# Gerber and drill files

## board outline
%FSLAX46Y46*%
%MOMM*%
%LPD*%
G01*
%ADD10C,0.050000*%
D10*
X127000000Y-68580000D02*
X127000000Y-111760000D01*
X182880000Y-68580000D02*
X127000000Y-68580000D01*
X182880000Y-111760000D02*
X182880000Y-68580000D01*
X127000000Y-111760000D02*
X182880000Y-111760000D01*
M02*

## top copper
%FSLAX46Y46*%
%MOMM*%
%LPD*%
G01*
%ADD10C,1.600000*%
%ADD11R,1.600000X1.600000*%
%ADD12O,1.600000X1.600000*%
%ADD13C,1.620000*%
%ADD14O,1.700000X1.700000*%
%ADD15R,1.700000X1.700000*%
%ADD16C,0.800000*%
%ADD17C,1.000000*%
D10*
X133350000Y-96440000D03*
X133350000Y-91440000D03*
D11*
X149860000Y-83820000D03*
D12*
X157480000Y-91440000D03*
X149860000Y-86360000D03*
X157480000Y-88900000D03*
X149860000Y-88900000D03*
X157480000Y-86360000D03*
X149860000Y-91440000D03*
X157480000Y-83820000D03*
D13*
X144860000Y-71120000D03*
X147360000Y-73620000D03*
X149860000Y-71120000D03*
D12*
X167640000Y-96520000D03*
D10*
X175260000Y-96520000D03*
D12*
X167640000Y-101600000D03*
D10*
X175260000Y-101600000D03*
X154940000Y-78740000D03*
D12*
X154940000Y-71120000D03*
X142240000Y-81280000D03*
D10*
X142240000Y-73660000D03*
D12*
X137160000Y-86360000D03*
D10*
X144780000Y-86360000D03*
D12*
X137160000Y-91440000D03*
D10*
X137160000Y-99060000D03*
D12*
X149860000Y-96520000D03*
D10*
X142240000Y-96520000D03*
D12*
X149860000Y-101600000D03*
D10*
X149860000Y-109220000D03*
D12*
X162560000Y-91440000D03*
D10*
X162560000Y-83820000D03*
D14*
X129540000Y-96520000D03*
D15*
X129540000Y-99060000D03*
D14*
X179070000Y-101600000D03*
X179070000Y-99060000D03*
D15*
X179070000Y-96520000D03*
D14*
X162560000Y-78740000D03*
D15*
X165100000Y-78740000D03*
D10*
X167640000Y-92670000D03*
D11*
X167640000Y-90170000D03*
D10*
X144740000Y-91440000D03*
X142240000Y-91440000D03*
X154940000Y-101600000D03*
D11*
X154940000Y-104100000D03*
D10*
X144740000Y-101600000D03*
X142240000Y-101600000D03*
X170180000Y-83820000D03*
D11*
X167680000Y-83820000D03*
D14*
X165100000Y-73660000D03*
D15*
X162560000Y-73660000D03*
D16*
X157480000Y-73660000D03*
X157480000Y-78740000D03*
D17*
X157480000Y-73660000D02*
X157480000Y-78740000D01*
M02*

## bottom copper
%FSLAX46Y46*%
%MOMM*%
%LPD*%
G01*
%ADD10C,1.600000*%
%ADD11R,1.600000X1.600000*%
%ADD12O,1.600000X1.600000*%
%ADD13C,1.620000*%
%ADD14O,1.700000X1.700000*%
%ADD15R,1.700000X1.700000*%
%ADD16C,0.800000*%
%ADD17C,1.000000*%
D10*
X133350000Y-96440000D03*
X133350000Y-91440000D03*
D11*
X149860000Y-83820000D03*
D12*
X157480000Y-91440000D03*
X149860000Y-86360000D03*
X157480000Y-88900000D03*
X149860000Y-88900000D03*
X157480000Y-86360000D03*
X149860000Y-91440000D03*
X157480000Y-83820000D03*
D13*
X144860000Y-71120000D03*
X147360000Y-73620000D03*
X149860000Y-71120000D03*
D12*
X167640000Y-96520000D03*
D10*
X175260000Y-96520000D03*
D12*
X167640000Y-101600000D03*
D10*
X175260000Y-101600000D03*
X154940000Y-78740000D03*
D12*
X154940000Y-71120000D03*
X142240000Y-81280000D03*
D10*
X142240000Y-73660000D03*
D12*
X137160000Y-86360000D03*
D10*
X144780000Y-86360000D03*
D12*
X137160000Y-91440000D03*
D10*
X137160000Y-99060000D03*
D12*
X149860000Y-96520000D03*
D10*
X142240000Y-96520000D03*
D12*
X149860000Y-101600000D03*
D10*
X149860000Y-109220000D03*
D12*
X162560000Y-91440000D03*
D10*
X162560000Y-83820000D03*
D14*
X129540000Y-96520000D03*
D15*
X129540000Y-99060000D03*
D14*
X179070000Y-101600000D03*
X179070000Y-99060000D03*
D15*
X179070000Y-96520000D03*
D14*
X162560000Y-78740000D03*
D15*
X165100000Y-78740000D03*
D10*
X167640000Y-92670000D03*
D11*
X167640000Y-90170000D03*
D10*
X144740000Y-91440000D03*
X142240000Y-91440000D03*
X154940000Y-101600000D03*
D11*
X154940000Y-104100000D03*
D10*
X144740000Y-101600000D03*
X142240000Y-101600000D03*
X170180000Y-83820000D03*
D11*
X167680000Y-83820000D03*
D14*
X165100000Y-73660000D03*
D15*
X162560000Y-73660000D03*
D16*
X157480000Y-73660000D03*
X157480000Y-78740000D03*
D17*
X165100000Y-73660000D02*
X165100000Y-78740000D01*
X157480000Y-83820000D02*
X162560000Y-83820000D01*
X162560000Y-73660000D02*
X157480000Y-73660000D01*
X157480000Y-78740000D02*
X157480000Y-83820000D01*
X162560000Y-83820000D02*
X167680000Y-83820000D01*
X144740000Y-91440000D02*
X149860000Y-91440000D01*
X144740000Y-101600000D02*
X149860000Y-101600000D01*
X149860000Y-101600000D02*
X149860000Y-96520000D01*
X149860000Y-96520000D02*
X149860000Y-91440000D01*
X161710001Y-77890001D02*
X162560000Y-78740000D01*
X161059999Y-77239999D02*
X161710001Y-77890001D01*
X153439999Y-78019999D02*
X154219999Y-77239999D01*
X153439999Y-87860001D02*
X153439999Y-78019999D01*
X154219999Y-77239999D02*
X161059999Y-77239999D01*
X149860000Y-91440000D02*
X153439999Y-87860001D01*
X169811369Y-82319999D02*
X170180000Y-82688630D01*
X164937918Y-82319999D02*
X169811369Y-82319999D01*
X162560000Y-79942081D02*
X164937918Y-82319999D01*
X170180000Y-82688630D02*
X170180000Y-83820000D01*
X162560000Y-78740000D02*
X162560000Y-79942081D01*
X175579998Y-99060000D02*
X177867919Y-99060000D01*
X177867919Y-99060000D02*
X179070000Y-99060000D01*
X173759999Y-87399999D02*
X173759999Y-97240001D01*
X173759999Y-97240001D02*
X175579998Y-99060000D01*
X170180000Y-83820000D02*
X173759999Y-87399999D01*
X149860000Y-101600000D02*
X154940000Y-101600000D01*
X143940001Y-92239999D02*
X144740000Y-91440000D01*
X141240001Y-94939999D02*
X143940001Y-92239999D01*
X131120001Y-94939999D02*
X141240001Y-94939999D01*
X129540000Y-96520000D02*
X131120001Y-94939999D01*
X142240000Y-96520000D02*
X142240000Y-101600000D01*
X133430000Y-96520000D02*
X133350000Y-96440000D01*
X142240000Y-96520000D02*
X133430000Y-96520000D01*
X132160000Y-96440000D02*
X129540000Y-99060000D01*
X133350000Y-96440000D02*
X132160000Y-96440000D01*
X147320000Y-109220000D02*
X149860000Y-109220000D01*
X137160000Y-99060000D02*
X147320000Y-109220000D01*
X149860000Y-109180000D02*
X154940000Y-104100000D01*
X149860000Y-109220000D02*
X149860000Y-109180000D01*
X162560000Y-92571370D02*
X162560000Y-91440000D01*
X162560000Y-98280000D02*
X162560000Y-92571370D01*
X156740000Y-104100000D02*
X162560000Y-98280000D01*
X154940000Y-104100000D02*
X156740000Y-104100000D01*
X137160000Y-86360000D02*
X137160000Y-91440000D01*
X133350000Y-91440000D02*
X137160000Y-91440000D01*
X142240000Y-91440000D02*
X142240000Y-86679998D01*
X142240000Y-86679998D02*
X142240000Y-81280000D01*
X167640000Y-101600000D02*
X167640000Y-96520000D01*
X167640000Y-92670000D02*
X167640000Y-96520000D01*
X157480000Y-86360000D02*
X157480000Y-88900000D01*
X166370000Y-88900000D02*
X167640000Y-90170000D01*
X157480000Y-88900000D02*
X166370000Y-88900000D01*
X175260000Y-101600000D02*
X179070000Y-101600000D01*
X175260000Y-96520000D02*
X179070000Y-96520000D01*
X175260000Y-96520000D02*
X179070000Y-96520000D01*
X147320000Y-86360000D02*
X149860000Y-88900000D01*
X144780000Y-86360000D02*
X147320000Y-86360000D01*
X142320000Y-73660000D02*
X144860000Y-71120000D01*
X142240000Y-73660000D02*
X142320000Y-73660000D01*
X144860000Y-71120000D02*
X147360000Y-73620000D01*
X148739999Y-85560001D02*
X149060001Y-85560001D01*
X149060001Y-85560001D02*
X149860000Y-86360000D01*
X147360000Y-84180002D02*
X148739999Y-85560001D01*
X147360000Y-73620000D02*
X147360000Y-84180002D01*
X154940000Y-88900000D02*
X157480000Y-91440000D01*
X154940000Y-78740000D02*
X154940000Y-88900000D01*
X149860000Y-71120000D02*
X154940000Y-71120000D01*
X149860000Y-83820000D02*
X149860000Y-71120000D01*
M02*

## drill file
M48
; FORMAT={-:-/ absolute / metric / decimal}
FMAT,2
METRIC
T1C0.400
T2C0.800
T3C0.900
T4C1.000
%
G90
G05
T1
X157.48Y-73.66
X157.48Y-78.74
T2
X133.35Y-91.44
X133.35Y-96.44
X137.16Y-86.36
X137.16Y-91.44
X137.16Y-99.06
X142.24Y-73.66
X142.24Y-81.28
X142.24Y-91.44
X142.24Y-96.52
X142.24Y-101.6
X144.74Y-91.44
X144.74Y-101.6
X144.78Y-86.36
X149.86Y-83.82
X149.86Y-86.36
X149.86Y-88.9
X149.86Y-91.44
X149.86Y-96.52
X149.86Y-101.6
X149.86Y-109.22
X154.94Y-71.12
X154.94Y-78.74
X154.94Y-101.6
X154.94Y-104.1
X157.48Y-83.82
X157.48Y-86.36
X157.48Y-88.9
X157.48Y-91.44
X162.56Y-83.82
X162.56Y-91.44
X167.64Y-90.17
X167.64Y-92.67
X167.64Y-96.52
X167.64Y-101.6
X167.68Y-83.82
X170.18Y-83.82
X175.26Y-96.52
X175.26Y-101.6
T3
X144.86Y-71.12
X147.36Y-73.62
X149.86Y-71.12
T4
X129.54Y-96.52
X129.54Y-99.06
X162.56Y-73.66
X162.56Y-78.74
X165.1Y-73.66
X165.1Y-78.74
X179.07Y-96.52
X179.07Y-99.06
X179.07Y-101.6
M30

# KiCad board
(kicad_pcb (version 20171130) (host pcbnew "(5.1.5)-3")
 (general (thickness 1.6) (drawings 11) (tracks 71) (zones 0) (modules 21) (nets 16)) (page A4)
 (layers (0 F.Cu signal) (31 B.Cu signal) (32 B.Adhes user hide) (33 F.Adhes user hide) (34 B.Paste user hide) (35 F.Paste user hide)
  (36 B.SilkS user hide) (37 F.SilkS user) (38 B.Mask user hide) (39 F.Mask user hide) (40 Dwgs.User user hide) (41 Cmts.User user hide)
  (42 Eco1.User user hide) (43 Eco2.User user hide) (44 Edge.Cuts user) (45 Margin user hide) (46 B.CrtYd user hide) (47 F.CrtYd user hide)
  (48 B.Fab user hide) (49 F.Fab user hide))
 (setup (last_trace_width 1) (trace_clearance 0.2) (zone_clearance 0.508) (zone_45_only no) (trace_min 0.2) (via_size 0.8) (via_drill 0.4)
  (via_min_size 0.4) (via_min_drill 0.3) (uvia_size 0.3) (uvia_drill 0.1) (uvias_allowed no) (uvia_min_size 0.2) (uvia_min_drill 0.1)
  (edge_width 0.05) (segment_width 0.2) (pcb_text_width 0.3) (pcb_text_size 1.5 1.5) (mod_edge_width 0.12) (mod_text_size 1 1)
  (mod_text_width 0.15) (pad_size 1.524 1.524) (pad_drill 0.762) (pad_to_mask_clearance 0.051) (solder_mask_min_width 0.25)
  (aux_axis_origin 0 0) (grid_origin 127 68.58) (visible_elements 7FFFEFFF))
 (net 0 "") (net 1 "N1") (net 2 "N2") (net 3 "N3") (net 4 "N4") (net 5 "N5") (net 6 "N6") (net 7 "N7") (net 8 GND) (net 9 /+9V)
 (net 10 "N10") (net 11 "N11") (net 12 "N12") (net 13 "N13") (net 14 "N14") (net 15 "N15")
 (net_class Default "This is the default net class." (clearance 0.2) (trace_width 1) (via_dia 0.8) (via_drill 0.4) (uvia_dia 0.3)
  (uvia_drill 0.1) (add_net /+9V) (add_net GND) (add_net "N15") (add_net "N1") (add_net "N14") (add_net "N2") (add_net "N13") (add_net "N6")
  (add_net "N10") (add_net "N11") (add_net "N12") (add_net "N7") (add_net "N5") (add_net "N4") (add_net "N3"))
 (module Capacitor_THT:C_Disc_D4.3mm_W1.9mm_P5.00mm (layer F.Cu) (at 133.35 91.44 270)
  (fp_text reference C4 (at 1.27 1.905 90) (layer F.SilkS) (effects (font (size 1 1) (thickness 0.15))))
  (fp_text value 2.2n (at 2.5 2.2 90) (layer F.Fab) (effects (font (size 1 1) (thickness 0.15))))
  (pad 2 thru_hole circle (at 5 0 270) (size 1.6 1.6) (drill 0.8) (layers *.Cu *.Mask) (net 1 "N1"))
  (pad 1 thru_hole circle (at 0 0 270) (size 1.6 1.6) (drill 0.8) (layers *.Cu *.Mask) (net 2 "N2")))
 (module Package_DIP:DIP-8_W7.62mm (layer F.Cu) (at 149.86 83.82)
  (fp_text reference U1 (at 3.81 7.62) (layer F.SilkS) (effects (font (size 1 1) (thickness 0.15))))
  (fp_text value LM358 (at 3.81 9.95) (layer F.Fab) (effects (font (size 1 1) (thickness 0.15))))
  (pad 1 thru_hole rect (at 0 0) (size 1.6 1.6) (drill 0.8) (layers *.Cu *.Mask) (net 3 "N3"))
  (pad 5 thru_hole oval (at 7.62 7.62) (size 1.6 1.6) (drill 0.8) (layers *.Cu *.Mask) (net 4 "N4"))
  (pad 2 thru_hole oval (at 0 2.54) (size 1.6 1.6) (drill 0.8) (layers *.Cu *.Mask) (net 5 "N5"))
  (pad 6 thru_hole oval (at 7.62 5.08) (size 1.6 1.6) (drill 0.8) (layers *.Cu *.Mask) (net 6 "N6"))
  (pad 3 thru_hole oval (at 0 5.08) (size 1.6 1.6) (drill 0.8) (layers *.Cu *.Mask) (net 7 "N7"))
  (pad 7 thru_hole oval (at 7.62 2.54) (size 1.6 1.6) (drill 0.8) (layers *.Cu *.Mask) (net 6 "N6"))
  (pad 4 thru_hole oval (at 0 7.62) (size 1.6 1.6) (drill 0.8) (layers *.Cu *.Mask) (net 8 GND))
  (pad 8 thru_hole oval (at 7.62 0) (size 1.6 1.6) (drill 0.8) (layers *.Cu *.Mask) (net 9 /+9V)))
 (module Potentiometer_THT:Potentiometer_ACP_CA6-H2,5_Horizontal (layer F.Cu) (at 149.86 71.12 270)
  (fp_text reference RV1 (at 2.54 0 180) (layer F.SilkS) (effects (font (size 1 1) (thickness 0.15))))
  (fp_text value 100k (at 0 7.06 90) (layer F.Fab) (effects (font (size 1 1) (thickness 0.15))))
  (pad 3 thru_hole circle (at 0 5 270) (size 1.62 1.62) (drill 0.9) (layers *.Cu *.Mask) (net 5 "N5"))
  (pad 2 thru_hole circle (at 2.5 2.5 270) (size 1.62 1.62) (drill 0.9) (layers *.Cu *.Mask) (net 5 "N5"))
  (pad 1 thru_hole circle (at 0 0 270) (size 1.62 1.62) (drill 0.9) (layers *.Cu *.Mask) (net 3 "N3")))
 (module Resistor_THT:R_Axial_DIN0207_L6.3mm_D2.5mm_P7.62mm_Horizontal (layer F.Cu) (at 175.26 96.52 180)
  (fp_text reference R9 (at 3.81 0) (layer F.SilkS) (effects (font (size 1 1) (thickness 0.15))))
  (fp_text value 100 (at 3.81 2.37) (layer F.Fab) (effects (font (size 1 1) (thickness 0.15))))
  (pad 2 thru_hole oval (at 7.62 0 180) (size 1.6 1.6) (drill 0.8) (layers *.Cu *.Mask) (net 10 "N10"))
  (pad 1 thru_hole circle (at 0 0 180) (size 1.6 1.6) (drill 0.8) (layers *.Cu *.Mask) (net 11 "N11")))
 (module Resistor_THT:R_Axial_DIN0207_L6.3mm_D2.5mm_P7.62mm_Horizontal (layer F.Cu) (at 175.26 101.6 180)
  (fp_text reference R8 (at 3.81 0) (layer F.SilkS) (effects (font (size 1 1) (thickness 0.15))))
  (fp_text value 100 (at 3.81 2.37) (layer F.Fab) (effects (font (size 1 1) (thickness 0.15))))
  (pad 2 thru_hole oval (at 7.62 0 180) (size 1.6 1.6) (drill 0.8) (layers *.Cu *.Mask) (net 10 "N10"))
  (pad 1 thru_hole circle (at 0 0 180) (size 1.6 1.6) (drill 0.8) (layers *.Cu *.Mask) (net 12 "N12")))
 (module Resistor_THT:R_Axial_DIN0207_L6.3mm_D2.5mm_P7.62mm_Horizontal (layer F.Cu) (at 154.94 78.74 90)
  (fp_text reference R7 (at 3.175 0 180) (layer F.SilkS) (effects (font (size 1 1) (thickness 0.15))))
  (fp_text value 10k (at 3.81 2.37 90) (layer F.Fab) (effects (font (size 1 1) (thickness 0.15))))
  (pad 1 thru_hole circle (at 0 0 90) (size 1.6 1.6) (drill 0.8) (layers *.Cu *.Mask) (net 4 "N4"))
  (pad 2 thru_hole oval (at 7.62 0 90) (size 1.6 1.6) (drill 0.8) (layers *.Cu *.Mask) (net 3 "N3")))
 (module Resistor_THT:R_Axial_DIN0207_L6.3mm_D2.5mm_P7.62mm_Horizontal (layer F.Cu) (at 142.24 73.66 270)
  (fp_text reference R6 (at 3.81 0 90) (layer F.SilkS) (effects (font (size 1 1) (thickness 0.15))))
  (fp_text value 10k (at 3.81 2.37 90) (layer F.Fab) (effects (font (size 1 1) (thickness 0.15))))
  (pad 2 thru_hole oval (at 7.62 0 270) (size 1.6 1.6) (drill 0.8) (layers *.Cu *.Mask) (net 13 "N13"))
  (pad 1 thru_hole circle (at 0 0 270) (size 1.6 1.6) (drill 0.8) (layers *.Cu *.Mask) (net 5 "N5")))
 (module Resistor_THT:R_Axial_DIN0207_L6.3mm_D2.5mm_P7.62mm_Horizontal (layer F.Cu) (at 144.78 86.36 180)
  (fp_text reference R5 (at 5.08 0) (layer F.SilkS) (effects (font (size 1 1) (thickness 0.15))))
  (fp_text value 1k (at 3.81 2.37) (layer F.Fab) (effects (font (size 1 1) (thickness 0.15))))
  (pad 2 thru_hole oval (at 7.62 0 180) (size 1.6 1.6) (drill 0.8) (layers *.Cu *.Mask) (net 2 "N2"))
  (pad 1 thru_hole circle (at 0 0 180) (size 1.6 1.6) (drill 0.8) (layers *.Cu *.Mask) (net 7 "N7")))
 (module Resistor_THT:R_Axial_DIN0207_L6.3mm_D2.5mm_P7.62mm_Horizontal (layer F.Cu) (at 137.16 99.06 90)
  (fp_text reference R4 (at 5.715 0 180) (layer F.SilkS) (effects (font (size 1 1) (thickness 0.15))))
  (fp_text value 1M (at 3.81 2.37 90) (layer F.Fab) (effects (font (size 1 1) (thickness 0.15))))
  (pad 2 thru_hole oval (at 7.62 0 90) (size 1.6 1.6) (drill 0.8) (layers *.Cu *.Mask) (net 2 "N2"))
  (pad 1 thru_hole circle (at 0 0 90) (size 1.6 1.6) (drill 0.8) (layers *.Cu *.Mask) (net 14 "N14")))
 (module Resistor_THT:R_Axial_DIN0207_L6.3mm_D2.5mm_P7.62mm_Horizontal (layer F.Cu) (at 142.24 96.52)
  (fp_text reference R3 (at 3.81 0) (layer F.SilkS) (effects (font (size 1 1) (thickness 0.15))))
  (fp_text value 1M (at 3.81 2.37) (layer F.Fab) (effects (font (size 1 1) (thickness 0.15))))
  (pad 2 thru_hole oval (at 7.62 0) (size 1.6 1.6) (drill 0.8) (layers *.Cu *.Mask) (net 8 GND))
  (pad 1 thru_hole circle (at 0 0) (size 1.6 1.6) (drill 0.8) (layers *.Cu *.Mask) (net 1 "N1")))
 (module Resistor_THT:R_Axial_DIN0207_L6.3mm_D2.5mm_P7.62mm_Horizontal (layer F.Cu) (at 149.86 109.22 90)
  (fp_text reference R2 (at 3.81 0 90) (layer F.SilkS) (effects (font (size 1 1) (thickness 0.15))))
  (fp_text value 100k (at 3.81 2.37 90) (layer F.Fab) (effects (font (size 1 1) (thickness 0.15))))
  (pad 2 thru_hole oval (at 7.62 0 90) (size 1.6 1.6) (drill 0.8) (layers *.Cu *.Mask) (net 8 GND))
  (pad 1 thru_hole circle (at 0 0 90) (size 1.6 1.6) (drill 0.8) (layers *.Cu *.Mask) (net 14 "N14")))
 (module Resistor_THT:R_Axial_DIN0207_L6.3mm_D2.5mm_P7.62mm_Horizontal (layer F.Cu) (at 162.56 83.82 270)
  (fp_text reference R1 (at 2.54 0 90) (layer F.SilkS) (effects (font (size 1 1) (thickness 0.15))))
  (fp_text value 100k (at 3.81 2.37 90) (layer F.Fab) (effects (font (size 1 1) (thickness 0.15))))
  (pad 2 thru_hole oval (at 7.62 0 270) (size 1.6 1.6) (drill 0.8) (layers *.Cu *.Mask) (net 14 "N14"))
  (pad 1 thru_hole circle (at 0 0 270) (size 1.6 1.6) (drill 0.8) (layers *.Cu *.Mask) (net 9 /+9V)))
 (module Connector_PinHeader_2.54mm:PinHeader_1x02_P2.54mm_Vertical (layer F.Cu) (at 129.54 99.06 180)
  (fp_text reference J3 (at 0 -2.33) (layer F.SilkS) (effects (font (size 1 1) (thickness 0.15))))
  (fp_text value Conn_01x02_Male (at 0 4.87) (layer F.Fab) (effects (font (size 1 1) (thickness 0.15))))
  (pad 2 thru_hole oval (at 0 2.54 180) (size 1.7 1.7) (drill 1) (layers *.Cu *.Mask) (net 8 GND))
  (pad 1 thru_hole rect (at 0 0 180) (size 1.7 1.7) (drill 1) (layers *.Cu *.Mask) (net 1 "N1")))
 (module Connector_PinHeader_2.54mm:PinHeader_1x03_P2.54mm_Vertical (layer F.Cu) (at 179.07 96.52)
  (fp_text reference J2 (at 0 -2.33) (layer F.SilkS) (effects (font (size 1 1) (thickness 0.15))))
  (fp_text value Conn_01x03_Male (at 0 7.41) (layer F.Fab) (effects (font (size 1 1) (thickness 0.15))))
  (pad 3 thru_hole oval (at 0 5.08) (size 1.7 1.7) (drill 1) (layers *.Cu *.Mask) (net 12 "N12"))
  (pad 2 thru_hole oval (at 0 2.54) (size 1.7 1.7) (drill 1) (layers *.Cu *.Mask) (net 8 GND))
  (pad 1 thru_hole rect (at 0 0) (size 1.7 1.7) (drill 1) (layers *.Cu *.Mask) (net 11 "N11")))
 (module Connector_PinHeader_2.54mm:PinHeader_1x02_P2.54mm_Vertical (layer F.Cu) (at 165.1 78.74 270)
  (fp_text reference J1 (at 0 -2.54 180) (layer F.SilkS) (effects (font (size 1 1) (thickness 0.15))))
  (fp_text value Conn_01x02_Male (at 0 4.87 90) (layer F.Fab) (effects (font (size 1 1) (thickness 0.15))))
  (pad 2 thru_hole oval (at 0 2.54 270) (size 1.7 1.7) (drill 1) (layers *.Cu *.Mask) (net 8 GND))
  (pad 1 thru_hole rect (at 0 0 270) (size 1.7 1.7) (drill 1) (layers *.Cu *.Mask) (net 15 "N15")))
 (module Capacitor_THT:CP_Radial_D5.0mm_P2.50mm (layer F.Cu) (at 167.64 90.17 270)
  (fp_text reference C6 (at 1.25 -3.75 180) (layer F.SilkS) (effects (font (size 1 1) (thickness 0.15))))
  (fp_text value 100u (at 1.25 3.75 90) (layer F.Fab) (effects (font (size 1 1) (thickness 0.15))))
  (pad 2 thru_hole circle (at 2.5 0 270) (size 1.6 1.6) (drill 0.8) (layers *.Cu *.Mask) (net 10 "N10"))
  (pad 1 thru_hole rect (at 0 0 270) (size 1.6 1.6) (drill 0.8) (layers *.Cu *.Mask) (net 6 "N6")))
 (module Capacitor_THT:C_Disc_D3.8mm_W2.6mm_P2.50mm (layer F.Cu) (at 142.24 91.44)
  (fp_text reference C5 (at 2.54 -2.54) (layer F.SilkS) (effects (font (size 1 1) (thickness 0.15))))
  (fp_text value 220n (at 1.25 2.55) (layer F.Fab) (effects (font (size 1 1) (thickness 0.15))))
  (pad 2 thru_hole circle (at 2.5 0) (size 1.6 1.6) (drill 0.8) (layers *.Cu *.Mask) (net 8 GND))
  (pad 1 thru_hole circle (at 0 0) (size 1.6 1.6) (drill 0.8) (layers *.Cu *.Mask) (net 13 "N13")))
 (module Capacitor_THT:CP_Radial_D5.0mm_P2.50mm (layer F.Cu) (at 154.94 104.1 90)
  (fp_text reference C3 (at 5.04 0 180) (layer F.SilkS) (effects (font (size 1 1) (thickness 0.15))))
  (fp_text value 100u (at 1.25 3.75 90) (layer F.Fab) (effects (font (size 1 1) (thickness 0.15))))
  (pad 2 thru_hole circle (at 2.5 0 90) (size 1.6 1.6) (drill 0.8) (layers *.Cu *.Mask) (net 8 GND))
  (pad 1 thru_hole rect (at 0 0 90) (size 1.6 1.6) (drill 0.8) (layers *.Cu *.Mask) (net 14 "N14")))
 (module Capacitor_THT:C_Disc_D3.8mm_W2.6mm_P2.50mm (layer F.Cu) (at 142.24 101.6)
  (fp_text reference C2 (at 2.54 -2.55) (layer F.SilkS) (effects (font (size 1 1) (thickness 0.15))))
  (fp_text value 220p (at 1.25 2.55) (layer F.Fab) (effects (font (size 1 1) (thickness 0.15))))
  (pad 2 thru_hole circle (at 2.5 0) (size 1.6 1.6) (drill 0.8) (layers *.Cu *.Mask) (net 8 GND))
  (pad 1 thru_hole circle (at 0 0) (size 1.6 1.6) (drill 0.8) (layers *.Cu *.Mask) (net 1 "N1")))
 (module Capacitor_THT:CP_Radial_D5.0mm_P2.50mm (layer F.Cu) (at 167.68 83.82)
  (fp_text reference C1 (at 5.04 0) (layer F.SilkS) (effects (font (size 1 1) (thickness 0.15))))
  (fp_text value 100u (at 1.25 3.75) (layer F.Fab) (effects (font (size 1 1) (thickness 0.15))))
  (pad 2 thru_hole circle (at 2.5 0) (size 1.6 1.6) (drill 0.8) (layers *.Cu *.Mask) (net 8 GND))
  (pad 1 thru_hole rect (at 0 0) (size 1.6 1.6) (drill 0.8) (layers *.Cu *.Mask) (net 9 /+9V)))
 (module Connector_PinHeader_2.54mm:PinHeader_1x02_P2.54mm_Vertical (layer F.Cu) (at 162.56 73.66 90)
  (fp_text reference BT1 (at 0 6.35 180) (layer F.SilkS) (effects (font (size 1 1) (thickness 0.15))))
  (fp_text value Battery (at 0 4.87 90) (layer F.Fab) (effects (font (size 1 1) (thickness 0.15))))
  (pad 2 thru_hole oval (at 0 2.54 90) (size 1.7 1.7) (drill 1) (layers *.Cu *.Mask) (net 15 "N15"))
  (pad 1 thru_hole rect (at 0 0 90) (size 1.7 1.7) (drill 1) (layers *.Cu *.Mask) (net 9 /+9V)))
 (gr_line (start 127 68.58) (end 127 111.76) (layer Edge.Cuts) (width 0.05))
 (gr_line (start 182.88 68.58) (end 127 68.58) (layer Edge.Cuts) (width 0.05))
 (gr_line (start 182.88 111.76) (end 182.88 68.58) (layer Edge.Cuts) (width 0.05))
 (gr_line (start 127 111.76) (end 182.88 111.76) (layer Edge.Cuts) (width 0.05))
 (segment (start 165.1 73.66) (end 165.1 78.74) (width 1) (layer B.Cu) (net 15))
 (segment (start 157.48 83.82) (end 162.56 83.82) (width 1) (layer B.Cu) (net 9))
 (via (at 157.48 73.66) (size 0.8) (drill 0.4) (layers F.Cu B.Cu) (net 9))
 (segment (start 162.56 73.66) (end 157.48 73.66) (width 1) (layer B.Cu) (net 9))
 (via (at 157.48 78.74) (size 0.8) (drill 0.4) (layers F.Cu B.Cu) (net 9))
 (segment (start 157.48 73.66) (end 157.48 78.74) (width 1) (layer F.Cu) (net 9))
 (segment (start 157.48 78.74) (end 157.48 83.82) (width 1) (layer B.Cu) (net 9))
 (segment (start 162.56 83.82) (end 167.68 83.82) (width 1) (layer B.Cu) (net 9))
 (segment (start 144.74 91.44) (end 149.86 91.44) (width 1) (layer B.Cu) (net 8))
 (segment (start 144.74 101.6) (end 149.86 101.6) (width 1) (layer B.Cu) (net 8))
 (segment (start 149.86 101.6) (end 149.86 96.52) (width 1) (layer B.Cu) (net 8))
 (segment (start 149.86 96.52) (end 149.86 91.44) (width 1) (layer B.Cu) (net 8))
 (segment (start 161.710001 77.890001) (end 162.56 78.74) (width 1) (layer B.Cu) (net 8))
 (segment (start 161.059999 77.239999) (end 161.710001 77.890001) (width 1) (layer B.Cu) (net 8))
 (segment (start 153.439999 78.019999) (end 154.219999 77.239999) (width 1) (layer B.Cu) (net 8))
 (segment (start 153.439999 87.860001) (end 153.439999 78.019999) (width 1) (layer B.Cu) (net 8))
 (segment (start 154.219999 77.239999) (end 161.059999 77.239999) (width 1) (layer B.Cu) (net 8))
 (segment (start 149.86 91.44) (end 153.439999 87.860001) (width 1) (layer B.Cu) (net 8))
 (segment (start 169.811369 82.319999) (end 170.18 82.68863) (width 1) (layer B.Cu) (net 8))
 (segment (start 164.937918 82.319999) (end 169.811369 82.319999) (width 1) (layer B.Cu) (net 8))
 (segment (start 162.56 79.942081) (end 164.937918 82.319999) (width 1) (layer B.Cu) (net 8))
 (segment (start 170.18 82.68863) (end 170.18 83.82) (width 1) (layer B.Cu) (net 8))
 (segment (start 162.56 78.74) (end 162.56 79.942081) (width 1) (layer B.Cu) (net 8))
 (segment (start 175.579998 99.06) (end 177.867919 99.06) (width 1) (layer B.Cu) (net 8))
 (segment (start 177.867919 99.06) (end 179.07 99.06) (width 1) (layer B.Cu) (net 8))
 (segment (start 173.759999 87.399999) (end 173.759999 97.240001) (width 1) (layer B.Cu) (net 8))
 (segment (start 173.759999 97.240001) (end 175.579998 99.06) (width 1) (layer B.Cu) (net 8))
 (segment (start 170.18 83.82) (end 173.759999 87.399999) (width 1) (layer B.Cu) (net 8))
 (segment (start 149.86 101.6) (end 154.94 101.6) (width 1) (layer B.Cu) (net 8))
 (segment (start 143.940001 92.239999) (end 144.74 91.44) (width 1) (layer B.Cu) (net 8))
 (segment (start 141.240001 94.939999) (end 143.940001 92.239999) (width 1) (layer B.Cu) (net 8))
 (segment (start 131.120001 94.939999) (end 141.240001 94.939999) (width 1) (layer B.Cu) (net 8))
 (segment (start 129.54 96.52) (end 131.120001 94.939999) (width 1) (layer B.Cu) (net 8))
 (segment (start 142.24 96.52) (end 142.24 101.6) (width 1) (layer B.Cu) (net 1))
 (segment (start 133.43 96.52) (end 133.35 96.44) (width 1) (layer B.Cu) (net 1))
 (segment (start 142.24 96.52) (end 133.43 96.52) (width 1) (layer B.Cu) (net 1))
 (segment (start 132.16 96.44) (end 129.54 99.06) (width 1) (layer B.Cu) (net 1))
 (segment (start 133.35 96.44) (end 132.16 96.44) (width 1) (layer B.Cu) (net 1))
 (segment (start 147.32 109.22) (end 149.86 109.22) (width 1) (layer B.Cu) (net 14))
 (segment (start 137.16 99.06) (end 147.32 109.22) (width 1) (layer B.Cu) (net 14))
 (segment (start 149.86 109.18) (end 154.94 104.1) (width 1) (layer B.Cu) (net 14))
 (segment (start 149.86 109.22) (end 149.86 109.18) (width 1) (layer B.Cu) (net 14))
 (segment (start 162.56 92.57137) (end 162.56 91.44) (width 1) (layer B.Cu) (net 14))
 (segment (start 162.56 98.28) (end 162.56 92.57137) (width 1) (layer B.Cu) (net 14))
 (segment (start 156.74 104.1) (end 162.56 98.28) (width 1) (layer B.Cu) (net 14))
 (segment (start 154.94 104.1) (end 156.74 104.1) (width 1) (layer B.Cu) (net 14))
 (segment (start 137.16 86.36) (end 137.16 91.44) (width 1) (layer B.Cu) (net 2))
 (segment (start 133.35 91.44) (end 137.16 91.44) (width 1) (layer B.Cu) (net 2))
 (segment (start 142.24 91.44) (end 142.24 86.679998) (width 1) (layer B.Cu) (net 13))
 (segment (start 142.24 86.679998) (end 142.24 81.28) (width 1) (layer B.Cu) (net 13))
 (segment (start 167.64 101.6) (end 167.64 96.52) (width 1) (layer B.Cu) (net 10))
 (segment (start 167.64 92.67) (end 167.64 96.52) (width 1) (layer B.Cu) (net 10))
 (segment (start 157.48 86.36) (end 157.48 88.9) (width 1) (layer B.Cu) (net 6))
 (segment (start 166.37 88.9) (end 167.64 90.17) (width 1) (layer B.Cu) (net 6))
 (segment (start 157.48 88.9) (end 166.37 88.9) (width 1) (layer B.Cu) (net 6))
 (segment (start 175.26 101.6) (end 179.07 101.6) (width 1) (layer B.Cu) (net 12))
 (segment (start 175.26 96.52) (end 179.07 96.52) (width 1) (layer B.Cu) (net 11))
 (segment (start 175.26 96.52) (end 179.07 96.52) (width 1) (layer B.Cu) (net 11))
 (segment (start 147.32 86.36) (end 149.86 88.9) (width 1) (layer B.Cu) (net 7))
 (segment (start 144.78 86.36) (end 147.32 86.36) (width 1) (layer B.Cu) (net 7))
 (segment (start 142.32 73.66) (end 144.86 71.12) (width 1) (layer B.Cu) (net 5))
 (segment (start 142.24 73.66) (end 142.32 73.66) (width 1) (layer B.Cu) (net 5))
 (segment (start 144.86 71.12) (end 147.36 73.62) (width 1) (layer B.Cu) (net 5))
 (segment (start 148.739999 85.560001) (end 149.060001 85.560001) (width 1) (layer B.Cu) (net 5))
 (segment (start 149.060001 85.560001) (end 149.86 86.36) (width 1) (layer B.Cu) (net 5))
 (segment (start 147.36 84.180002) (end 148.739999 85.560001) (width 1) (layer B.Cu) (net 5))
 (segment (start 147.36 73.62) (end 147.36 84.180002) (width 1) (layer B.Cu) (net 5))
 (segment (start 154.94 88.9) (end 157.48 91.44) (width 1) (layer B.Cu) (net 4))
 (segment (start 154.94 78.74) (end 154.94 88.9) (width 1) (layer B.Cu) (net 4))
 (segment (start 149.86 71.12) (end 154.94 71.12) (width 1) (layer B.Cu) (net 3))
 (segment (start 149.86 83.82) (end 149.86 71.12) (width 1) (layer B.Cu) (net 3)))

